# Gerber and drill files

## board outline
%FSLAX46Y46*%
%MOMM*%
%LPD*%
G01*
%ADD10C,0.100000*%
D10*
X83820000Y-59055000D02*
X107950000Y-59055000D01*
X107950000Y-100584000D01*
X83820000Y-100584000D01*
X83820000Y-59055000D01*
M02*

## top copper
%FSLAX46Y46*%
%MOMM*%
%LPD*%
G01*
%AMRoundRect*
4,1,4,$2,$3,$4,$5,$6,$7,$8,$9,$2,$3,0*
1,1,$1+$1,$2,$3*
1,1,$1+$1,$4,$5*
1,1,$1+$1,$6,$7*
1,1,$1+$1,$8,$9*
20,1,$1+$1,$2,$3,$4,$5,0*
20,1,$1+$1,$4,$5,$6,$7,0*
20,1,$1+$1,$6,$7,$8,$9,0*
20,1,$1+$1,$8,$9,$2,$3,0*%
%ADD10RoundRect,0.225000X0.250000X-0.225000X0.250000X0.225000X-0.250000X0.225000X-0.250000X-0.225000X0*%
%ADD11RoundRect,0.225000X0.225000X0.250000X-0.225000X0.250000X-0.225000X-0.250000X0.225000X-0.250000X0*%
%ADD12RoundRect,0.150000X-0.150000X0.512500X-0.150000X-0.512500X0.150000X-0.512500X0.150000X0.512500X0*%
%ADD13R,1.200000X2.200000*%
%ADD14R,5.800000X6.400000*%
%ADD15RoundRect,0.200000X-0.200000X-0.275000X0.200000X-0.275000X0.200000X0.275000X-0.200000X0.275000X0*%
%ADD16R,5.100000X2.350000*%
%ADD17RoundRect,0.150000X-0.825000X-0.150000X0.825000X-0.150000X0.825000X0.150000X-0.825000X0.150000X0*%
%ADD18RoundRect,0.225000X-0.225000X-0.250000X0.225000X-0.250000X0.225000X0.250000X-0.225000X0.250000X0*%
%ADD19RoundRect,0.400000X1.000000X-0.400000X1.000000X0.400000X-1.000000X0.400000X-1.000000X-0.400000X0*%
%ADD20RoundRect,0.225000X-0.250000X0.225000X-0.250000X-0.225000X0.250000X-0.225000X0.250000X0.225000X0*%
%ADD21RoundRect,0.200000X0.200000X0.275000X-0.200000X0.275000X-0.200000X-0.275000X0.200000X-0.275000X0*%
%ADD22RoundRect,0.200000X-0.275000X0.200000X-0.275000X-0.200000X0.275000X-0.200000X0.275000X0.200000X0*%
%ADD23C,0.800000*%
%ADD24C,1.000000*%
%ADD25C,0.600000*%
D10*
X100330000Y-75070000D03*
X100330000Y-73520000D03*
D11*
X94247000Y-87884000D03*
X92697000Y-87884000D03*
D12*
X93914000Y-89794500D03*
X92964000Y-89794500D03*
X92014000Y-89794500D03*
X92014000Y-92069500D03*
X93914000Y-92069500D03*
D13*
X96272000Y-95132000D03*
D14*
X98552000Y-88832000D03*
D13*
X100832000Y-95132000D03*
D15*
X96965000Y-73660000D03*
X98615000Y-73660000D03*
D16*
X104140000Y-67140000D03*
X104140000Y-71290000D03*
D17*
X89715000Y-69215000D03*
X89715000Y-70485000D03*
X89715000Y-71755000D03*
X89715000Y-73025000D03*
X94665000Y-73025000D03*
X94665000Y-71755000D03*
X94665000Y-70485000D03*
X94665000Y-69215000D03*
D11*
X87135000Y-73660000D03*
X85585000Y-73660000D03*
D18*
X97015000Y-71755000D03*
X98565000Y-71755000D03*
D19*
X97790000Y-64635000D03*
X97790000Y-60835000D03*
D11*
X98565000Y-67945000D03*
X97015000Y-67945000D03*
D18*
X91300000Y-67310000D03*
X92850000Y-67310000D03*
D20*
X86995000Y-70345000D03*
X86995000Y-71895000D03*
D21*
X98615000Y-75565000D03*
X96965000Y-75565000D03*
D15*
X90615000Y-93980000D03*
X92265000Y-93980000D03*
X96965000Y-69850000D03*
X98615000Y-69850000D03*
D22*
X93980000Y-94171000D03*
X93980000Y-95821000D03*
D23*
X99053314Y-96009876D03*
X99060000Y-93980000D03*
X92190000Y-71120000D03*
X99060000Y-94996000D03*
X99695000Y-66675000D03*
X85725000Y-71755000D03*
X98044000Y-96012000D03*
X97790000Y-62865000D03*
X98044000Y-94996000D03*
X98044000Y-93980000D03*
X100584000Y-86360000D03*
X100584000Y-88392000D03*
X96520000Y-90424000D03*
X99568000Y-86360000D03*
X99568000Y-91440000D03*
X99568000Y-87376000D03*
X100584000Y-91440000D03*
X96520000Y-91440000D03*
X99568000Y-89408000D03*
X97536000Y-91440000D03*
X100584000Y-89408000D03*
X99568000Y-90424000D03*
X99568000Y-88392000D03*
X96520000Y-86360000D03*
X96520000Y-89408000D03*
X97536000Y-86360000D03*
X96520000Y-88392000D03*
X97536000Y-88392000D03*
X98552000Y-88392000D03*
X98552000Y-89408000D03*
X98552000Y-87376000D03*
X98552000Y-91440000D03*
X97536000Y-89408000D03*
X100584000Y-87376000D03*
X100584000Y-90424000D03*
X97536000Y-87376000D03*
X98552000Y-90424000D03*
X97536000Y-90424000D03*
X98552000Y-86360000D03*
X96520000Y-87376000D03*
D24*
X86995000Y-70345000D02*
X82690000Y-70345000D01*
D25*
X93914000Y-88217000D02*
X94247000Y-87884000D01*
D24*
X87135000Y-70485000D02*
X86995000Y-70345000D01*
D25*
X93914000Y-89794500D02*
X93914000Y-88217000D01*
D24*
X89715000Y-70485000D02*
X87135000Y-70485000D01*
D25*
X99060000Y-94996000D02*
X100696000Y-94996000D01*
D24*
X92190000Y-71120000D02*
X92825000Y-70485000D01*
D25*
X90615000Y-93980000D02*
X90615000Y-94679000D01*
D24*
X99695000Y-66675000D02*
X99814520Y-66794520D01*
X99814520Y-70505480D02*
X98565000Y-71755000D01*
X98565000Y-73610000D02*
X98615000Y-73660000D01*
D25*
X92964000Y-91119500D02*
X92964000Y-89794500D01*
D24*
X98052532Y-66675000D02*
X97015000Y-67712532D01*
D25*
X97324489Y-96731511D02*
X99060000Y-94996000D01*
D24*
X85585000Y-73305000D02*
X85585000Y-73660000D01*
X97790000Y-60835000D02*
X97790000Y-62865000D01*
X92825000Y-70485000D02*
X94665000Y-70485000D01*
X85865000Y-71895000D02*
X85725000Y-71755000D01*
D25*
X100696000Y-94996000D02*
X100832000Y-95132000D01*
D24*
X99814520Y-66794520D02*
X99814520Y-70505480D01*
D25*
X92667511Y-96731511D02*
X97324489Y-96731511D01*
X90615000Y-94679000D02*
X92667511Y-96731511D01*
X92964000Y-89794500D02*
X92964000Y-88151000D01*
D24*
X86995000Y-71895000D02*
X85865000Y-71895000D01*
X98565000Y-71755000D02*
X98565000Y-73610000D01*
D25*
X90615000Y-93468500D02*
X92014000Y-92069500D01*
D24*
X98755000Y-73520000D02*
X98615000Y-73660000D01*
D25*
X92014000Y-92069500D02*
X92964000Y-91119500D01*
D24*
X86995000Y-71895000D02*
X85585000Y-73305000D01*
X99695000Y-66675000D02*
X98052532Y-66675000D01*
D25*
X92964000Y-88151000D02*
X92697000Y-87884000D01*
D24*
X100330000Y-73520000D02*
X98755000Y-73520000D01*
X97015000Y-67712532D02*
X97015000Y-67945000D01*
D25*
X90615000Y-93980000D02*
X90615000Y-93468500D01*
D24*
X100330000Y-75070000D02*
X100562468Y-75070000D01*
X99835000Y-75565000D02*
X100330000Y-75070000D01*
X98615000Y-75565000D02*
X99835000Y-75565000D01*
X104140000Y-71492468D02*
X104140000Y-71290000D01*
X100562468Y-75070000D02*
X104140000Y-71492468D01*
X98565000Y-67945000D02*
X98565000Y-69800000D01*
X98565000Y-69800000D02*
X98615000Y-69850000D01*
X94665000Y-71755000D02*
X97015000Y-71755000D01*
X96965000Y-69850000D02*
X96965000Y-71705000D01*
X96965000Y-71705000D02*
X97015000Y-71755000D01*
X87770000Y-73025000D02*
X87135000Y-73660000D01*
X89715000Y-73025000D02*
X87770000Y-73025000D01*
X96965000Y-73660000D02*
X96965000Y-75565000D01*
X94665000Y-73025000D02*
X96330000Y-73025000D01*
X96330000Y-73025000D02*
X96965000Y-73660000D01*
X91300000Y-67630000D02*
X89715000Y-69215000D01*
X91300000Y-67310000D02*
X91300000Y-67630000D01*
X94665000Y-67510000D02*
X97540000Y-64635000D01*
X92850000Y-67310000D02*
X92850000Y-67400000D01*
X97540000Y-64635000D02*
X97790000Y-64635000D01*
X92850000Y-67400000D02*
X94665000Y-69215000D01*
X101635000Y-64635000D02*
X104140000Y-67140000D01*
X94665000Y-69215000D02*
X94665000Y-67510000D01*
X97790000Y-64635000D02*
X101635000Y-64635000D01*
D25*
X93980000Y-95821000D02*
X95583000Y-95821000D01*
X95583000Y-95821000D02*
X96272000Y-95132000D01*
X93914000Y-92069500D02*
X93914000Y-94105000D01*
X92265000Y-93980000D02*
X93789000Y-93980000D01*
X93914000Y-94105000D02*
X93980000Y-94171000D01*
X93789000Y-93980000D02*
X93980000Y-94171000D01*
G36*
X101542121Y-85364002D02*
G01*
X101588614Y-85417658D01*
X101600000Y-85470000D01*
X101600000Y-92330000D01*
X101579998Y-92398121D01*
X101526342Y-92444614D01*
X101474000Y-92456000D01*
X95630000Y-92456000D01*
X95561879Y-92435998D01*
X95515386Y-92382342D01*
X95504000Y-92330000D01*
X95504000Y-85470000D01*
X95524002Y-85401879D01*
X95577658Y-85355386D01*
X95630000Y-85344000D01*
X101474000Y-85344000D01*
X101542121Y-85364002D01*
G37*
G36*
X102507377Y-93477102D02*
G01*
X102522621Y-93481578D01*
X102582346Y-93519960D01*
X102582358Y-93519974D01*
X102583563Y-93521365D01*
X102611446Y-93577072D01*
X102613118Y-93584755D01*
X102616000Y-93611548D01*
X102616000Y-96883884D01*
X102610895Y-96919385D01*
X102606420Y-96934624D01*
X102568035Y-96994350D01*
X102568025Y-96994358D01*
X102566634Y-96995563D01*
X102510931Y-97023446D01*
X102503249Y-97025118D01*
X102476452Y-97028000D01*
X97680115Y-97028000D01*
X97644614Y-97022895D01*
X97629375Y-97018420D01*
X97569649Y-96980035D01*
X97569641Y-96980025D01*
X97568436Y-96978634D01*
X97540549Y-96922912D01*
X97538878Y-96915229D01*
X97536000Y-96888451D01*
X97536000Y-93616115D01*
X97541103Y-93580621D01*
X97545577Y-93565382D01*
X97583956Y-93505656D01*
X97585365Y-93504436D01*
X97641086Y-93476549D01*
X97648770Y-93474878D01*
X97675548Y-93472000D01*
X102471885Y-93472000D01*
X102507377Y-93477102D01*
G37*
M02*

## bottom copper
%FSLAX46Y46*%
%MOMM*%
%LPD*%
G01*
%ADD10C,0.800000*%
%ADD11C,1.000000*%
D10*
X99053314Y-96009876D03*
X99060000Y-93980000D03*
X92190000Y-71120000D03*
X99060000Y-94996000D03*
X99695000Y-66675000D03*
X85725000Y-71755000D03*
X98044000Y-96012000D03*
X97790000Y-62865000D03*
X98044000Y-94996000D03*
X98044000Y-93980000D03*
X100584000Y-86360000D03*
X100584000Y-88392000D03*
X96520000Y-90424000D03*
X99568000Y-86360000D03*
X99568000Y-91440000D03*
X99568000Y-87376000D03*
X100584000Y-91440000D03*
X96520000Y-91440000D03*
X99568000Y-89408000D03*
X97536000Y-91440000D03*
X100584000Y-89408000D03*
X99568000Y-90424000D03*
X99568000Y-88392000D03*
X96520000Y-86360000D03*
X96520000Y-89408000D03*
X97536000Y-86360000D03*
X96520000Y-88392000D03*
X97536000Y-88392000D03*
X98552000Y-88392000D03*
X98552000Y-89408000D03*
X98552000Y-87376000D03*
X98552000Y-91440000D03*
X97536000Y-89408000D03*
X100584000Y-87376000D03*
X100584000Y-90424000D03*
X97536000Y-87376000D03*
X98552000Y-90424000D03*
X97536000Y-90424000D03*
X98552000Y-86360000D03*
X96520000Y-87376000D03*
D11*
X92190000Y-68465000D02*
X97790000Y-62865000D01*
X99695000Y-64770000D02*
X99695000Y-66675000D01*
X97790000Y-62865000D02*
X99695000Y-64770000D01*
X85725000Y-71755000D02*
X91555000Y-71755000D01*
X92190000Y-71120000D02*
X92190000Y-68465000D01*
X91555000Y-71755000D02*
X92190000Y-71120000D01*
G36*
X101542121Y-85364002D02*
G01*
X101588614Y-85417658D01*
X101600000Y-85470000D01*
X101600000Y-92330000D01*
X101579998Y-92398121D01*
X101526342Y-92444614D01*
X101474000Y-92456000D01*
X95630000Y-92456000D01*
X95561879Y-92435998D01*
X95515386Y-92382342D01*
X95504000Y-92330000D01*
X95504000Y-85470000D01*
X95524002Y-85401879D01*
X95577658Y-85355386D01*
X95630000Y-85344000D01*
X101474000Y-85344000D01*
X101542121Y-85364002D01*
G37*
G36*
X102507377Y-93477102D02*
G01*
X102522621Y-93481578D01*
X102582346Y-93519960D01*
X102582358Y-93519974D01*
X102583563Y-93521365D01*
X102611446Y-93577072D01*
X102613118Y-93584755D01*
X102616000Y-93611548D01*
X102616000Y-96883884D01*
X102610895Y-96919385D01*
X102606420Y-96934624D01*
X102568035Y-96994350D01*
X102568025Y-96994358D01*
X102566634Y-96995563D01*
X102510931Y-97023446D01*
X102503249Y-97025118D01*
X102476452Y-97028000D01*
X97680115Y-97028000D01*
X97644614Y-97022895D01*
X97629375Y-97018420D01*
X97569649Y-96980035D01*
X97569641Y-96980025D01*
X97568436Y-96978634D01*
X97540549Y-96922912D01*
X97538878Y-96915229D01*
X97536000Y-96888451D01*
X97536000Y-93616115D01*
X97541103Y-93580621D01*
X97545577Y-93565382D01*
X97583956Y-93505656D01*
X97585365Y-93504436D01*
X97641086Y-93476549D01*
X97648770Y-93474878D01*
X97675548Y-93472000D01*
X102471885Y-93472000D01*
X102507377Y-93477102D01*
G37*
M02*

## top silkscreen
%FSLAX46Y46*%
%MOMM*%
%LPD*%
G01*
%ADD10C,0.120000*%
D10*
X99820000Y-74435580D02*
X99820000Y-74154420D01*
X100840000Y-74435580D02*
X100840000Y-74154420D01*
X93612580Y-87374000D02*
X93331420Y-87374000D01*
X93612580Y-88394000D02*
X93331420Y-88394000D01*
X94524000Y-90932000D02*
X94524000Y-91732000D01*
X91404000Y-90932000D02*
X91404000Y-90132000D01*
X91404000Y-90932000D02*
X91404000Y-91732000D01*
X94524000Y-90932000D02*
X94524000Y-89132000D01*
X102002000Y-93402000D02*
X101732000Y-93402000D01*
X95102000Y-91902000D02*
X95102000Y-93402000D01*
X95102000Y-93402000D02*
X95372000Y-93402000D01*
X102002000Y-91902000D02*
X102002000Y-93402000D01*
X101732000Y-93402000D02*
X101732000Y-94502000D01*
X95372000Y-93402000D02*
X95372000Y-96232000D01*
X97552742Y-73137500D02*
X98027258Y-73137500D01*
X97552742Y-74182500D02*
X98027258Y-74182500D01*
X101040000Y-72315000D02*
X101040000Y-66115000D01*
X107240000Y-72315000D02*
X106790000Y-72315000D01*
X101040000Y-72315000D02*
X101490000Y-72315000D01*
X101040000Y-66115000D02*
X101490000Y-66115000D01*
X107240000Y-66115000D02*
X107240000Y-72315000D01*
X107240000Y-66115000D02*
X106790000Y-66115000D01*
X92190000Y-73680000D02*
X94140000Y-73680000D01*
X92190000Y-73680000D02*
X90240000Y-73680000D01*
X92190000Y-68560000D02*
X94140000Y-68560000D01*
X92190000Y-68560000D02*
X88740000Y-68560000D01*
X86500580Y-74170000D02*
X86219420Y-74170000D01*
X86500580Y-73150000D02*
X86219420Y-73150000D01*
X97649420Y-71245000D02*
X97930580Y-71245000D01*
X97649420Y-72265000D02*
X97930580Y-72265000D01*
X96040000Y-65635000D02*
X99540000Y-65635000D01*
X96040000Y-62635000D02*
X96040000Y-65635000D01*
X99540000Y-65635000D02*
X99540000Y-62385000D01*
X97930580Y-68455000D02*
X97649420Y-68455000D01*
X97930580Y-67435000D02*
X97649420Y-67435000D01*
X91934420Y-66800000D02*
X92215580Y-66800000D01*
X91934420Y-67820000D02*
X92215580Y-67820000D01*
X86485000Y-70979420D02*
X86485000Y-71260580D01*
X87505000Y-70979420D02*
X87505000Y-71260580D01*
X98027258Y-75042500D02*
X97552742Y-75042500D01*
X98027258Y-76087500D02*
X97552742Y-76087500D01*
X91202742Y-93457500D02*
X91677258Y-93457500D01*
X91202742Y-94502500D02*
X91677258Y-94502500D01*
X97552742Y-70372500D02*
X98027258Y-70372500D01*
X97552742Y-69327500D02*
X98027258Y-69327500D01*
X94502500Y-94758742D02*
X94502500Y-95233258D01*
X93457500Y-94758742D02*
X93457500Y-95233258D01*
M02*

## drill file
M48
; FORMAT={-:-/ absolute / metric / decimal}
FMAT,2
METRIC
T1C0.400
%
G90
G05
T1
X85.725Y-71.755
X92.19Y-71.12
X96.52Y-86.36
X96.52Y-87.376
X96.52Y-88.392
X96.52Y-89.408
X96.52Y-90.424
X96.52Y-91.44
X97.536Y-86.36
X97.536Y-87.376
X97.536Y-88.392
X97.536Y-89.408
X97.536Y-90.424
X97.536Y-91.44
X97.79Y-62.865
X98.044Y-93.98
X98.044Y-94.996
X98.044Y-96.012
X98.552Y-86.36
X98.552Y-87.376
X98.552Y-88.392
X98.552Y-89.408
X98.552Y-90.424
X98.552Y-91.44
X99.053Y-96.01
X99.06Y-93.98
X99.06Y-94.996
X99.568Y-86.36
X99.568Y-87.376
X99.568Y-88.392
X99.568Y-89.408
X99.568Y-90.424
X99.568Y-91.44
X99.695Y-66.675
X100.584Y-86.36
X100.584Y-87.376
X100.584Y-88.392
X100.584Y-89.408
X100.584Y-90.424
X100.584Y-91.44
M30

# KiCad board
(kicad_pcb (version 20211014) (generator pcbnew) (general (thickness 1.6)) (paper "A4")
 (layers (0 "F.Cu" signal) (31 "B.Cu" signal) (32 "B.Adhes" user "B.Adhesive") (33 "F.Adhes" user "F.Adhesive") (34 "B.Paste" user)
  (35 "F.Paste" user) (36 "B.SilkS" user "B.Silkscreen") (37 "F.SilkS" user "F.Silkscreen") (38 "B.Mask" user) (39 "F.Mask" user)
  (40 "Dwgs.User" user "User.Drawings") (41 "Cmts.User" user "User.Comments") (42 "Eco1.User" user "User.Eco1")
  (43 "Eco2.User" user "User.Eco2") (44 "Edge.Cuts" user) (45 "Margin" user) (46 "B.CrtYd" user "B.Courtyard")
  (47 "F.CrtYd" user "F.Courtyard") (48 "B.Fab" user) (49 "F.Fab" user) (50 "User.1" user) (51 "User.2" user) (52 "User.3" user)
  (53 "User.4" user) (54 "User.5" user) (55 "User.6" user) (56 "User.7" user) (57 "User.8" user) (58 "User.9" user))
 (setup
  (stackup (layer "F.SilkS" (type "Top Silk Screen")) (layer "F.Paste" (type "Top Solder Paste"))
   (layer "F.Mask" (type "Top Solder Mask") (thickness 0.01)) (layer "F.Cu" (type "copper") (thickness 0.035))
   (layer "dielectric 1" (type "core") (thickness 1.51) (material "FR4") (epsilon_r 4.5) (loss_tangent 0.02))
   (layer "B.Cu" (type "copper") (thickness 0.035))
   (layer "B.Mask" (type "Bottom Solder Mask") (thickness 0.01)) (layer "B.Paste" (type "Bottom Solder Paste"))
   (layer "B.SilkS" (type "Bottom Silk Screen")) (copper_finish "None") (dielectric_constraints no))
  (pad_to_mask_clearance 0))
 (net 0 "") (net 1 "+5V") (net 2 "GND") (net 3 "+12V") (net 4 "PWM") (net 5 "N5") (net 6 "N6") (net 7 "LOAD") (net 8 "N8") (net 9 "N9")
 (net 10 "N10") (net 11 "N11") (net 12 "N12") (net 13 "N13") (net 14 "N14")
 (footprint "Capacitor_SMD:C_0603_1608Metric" (layer "F.Cu") (at 100.33 74.295 90)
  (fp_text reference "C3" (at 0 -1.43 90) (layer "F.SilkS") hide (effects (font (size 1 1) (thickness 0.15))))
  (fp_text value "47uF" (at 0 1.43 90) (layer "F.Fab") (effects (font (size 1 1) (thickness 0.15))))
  (fp_line (start -0.14058 -0.51) (end 0.14058 -0.51) (layer "F.SilkS") (width 0.12))
  (fp_line (start -0.14058 0.51) (end 0.14058 0.51) (layer "F.SilkS") (width 0.12))
  (pad "1" smd roundrect (at -0.775 0 90) (size 0.9 0.95) (layers "F.Cu" "F.Paste" "F.Mask") (roundrect_rratio 0.25) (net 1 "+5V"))
  (pad "2" smd roundrect (at 0.775 0 90) (size 0.9 0.95) (layers "F.Cu" "F.Paste" "F.Mask") (roundrect_rratio 0.25) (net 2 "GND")))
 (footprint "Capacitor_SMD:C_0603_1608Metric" (layer "F.Cu") (at 93.472 87.884 180)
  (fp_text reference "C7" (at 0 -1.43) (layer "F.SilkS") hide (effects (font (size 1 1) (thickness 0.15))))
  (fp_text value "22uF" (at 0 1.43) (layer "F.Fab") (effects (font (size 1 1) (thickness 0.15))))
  (fp_line (start -0.14058 0.51) (end 0.14058 0.51) (layer "F.SilkS") (width 0.12))
  (fp_line (start -0.14058 -0.51) (end 0.14058 -0.51) (layer "F.SilkS") (width 0.12))
  (pad "1" smd roundrect (at -0.775 0 180) (size 0.9 0.95) (layers "F.Cu" "F.Paste" "F.Mask") (roundrect_rratio 0.25) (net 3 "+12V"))
  (pad "2" smd roundrect (at 0.775 0 180) (size 0.9 0.95) (layers "F.Cu" "F.Paste" "F.Mask") (roundrect_rratio 0.25) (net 2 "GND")))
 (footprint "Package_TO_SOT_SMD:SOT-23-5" (layer "F.Cu") (at 92.964 90.932 -90)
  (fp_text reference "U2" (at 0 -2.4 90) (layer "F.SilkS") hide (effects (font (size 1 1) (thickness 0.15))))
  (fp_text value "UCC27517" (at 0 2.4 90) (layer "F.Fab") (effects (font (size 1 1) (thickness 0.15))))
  (fp_line (start 0 -1.56) (end 0.8 -1.56) (layer "F.SilkS") (width 0.12))
  (fp_line (start 0 1.56) (end -0.8 1.56) (layer "F.SilkS") (width 0.12))
  (fp_line (start 0 1.56) (end 0.8 1.56) (layer "F.SilkS") (width 0.12))
  (fp_line (start 0 -1.56) (end -1.8 -1.56) (layer "F.SilkS") (width 0.12))
  (pad "1" smd roundrect (at -1.1375 -0.95 270) (size 1.325 0.6) (layers "F.Cu" "F.Paste" "F.Mask") (roundrect_rratio 0.25) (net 3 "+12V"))
  (pad "2" smd roundrect (at -1.1375 0 270) (size 1.325 0.6) (layers "F.Cu" "F.Paste" "F.Mask") (roundrect_rratio 0.25) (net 2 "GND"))
  (pad "3" smd roundrect (at -1.1375 0.95 270) (size 1.325 0.6) (layers "F.Cu" "F.Paste" "F.Mask") (roundrect_rratio 0.25) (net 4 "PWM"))
  (pad "4" smd roundrect (at 1.1375 0.95 270) (size 1.325 0.6) (layers "F.Cu" "F.Paste" "F.Mask") (roundrect_rratio 0.25) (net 2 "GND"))
  (pad "5" smd roundrect (at 1.1375 -0.95 270) (size 1.325 0.6) (layers "F.Cu" "F.Paste" "F.Mask") (roundrect_rratio 0.25) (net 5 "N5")))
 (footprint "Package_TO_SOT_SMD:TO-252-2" (layer "F.Cu") (at 98.552 90.932 90)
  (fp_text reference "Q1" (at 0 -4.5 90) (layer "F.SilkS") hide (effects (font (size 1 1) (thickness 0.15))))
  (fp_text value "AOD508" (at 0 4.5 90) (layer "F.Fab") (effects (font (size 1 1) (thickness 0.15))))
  (fp_line (start -2.47 3.45) (end -2.47 3.18) (layer "F.SilkS") (width 0.12))
  (fp_line (start -0.97 -3.45) (end -2.47 -3.45) (layer "F.SilkS") (width 0.12))
  (fp_line (start -2.47 -3.45) (end -2.47 -3.18) (layer "F.SilkS") (width 0.12))
  (fp_line (start -0.97 3.45) (end -2.47 3.45) (layer "F.SilkS") (width 0.12))
  (fp_line (start -2.47 3.18) (end -3.57 3.18) (layer "F.SilkS") (width 0.12))
  (fp_line (start -2.47 -3.18) (end -5.3 -3.18) (layer "F.SilkS") (width 0.12))
  (pad "" smd rect (at 0.425 1.525 90) (size 3.05 2.75) (layers "F.Paste"))
  (pad "" smd rect (at 3.775 1.525 90) (size 3.05 2.75) (layers "F.Paste"))
  (pad "" smd rect (at 3.775 -1.525 90) (size 3.05 2.75) (layers "F.Paste"))
  (pad "" smd rect (at 0.425 -1.525 90) (size 3.05 2.75) (layers "F.Paste"))
  (pad "1" smd rect (at -4.2 -2.28 90) (size 2.2 1.2) (layers "F.Cu" "F.Paste" "F.Mask") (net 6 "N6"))
  (pad "2" smd rect (at 2.1 0 90) (size 6.4 5.8) (layers "F.Cu" "F.Mask") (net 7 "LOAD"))
  (pad "3" smd rect (at -4.2 2.28 90) (size 2.2 1.2) (layers "F.Cu" "F.Paste" "F.Mask") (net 2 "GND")))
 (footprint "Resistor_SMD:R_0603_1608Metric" (layer "F.Cu") (at 97.79 73.66)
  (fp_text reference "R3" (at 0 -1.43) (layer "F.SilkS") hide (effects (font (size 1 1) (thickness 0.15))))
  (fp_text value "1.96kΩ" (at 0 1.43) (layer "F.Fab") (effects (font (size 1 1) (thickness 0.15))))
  (fp_line (start -0.237258 -0.5225) (end 0.237258 -0.5225) (layer "F.SilkS") (width 0.12))
  (fp_line (start -0.237258 0.5225) (end 0.237258 0.5225) (layer "F.SilkS") (width 0.12))
  (pad "1" smd roundrect (at -0.825 0) (size 0.8 0.95) (layers "F.Cu" "F.Paste" "F.Mask") (roundrect_rratio 0.25) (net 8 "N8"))
  (pad "2" smd roundrect (at 0.825 0) (size 0.8 0.95) (layers "F.Cu" "F.Paste" "F.Mask") (roundrect_rratio 0.25) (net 2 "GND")))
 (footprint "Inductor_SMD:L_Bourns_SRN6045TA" (layer "F.Cu") (at 104.14 69.215 -90)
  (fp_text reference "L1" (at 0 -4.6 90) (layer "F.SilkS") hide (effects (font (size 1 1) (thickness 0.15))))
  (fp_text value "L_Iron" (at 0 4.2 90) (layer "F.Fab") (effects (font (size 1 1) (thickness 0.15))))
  (fp_line (start 3.1 3.1) (end -3.1 3.1) (layer "F.SilkS") (width 0.12))
  (fp_line (start 3.1 -3.1) (end 3.1 -2.65) (layer "F.SilkS") (width 0.12))
  (fp_line (start 3.1 3.1) (end 3.1 2.65) (layer "F.SilkS") (width 0.12))
  (fp_line (start -3.1 3.1) (end -3.1 2.65) (layer "F.SilkS") (width 0.12))
  (fp_line (start -3.1 -3.1) (end 3.1 -3.1) (layer "F.SilkS") (width 0.12))
  (fp_line (start -3.1 -3.1) (end -3.1 -2.65) (layer "F.SilkS") (width 0.12))
  (pad "1" smd rect (at -2.075 0 270) (size 2.35 5.1) (layers "F.Cu" "F.Paste" "F.Mask") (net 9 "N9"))
  (pad "2" smd rect (at 2.075 0 270) (size 2.35 5.1) (layers "F.Cu" "F.Paste" "F.Mask") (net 1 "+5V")))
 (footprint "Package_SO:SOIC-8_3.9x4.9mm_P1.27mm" (layer "F.Cu") (at 92.19 71.12)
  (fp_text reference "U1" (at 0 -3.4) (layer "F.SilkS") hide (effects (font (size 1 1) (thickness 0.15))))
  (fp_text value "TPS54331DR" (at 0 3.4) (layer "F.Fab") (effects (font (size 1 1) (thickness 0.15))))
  (fp_line (start 0 2.56) (end 1.95 2.56) (layer "F.SilkS") (width 0.12))
  (fp_line (start 0 2.56) (end -1.95 2.56) (layer "F.SilkS") (width 0.12))
  (fp_line (start 0 -2.56) (end 1.95 -2.56) (layer "F.SilkS") (width 0.12))
  (fp_line (start 0 -2.56) (end -3.45 -2.56) (layer "F.SilkS") (width 0.12))
  (pad "1" smd roundrect (at -2.475 -1.905) (size 1.95 0.6) (layers "F.Cu" "F.Paste" "F.Mask") (roundrect_rratio 0.25) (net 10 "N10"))
  (pad "2" smd roundrect (at -2.475 -0.635) (size 1.95 0.6) (layers "F.Cu" "F.Paste" "F.Mask") (roundrect_rratio 0.25) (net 3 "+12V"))
  (pad "3" smd roundrect (at -2.475 0.635) (size 1.95 0.6) (layers "F.Cu" "F.Paste" "F.Mask") (roundrect_rratio 0.25) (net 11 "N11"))
  (pad "4" smd roundrect (at -2.475 1.905) (size 1.95 0.6) (layers "F.Cu" "F.Paste" "F.Mask") (roundrect_rratio 0.25) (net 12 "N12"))
  (pad "5" smd roundrect (at 2.475 1.905) (size 1.95 0.6) (layers "F.Cu" "F.Paste" "F.Mask") (roundrect_rratio 0.25) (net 8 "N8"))
  (pad "6" smd roundrect (at 2.475 0.635) (size 1.95 0.6) (layers "F.Cu" "F.Paste" "F.Mask") (roundrect_rratio 0.25) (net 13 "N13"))
  (pad "7" smd roundrect (at 2.475 -0.635) (size 1.95 0.6) (layers "F.Cu" "F.Paste" "F.Mask") (roundrect_rratio 0.25) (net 2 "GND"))
  (pad "8" smd roundrect (at 2.475 -1.905) (size 1.95 0.6) (layers "F.Cu" "F.Paste" "F.Mask") (roundrect_rratio 0.25) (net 9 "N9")))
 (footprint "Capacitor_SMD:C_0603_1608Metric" (layer "F.Cu") (at 86.36 73.66 180)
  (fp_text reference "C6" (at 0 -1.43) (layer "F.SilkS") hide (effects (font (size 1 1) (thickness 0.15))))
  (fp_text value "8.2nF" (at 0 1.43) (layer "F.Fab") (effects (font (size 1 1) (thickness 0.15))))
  (fp_line (start -0.14058 -0.51) (end 0.14058 -0.51) (layer "F.SilkS") (width 0.12))
  (fp_line (start -0.14058 0.51) (end 0.14058 0.51) (layer "F.SilkS") (width 0.12))
  (pad "1" smd roundrect (at -0.775 0 180) (size 0.9 0.95) (layers "F.Cu" "F.Paste" "F.Mask") (roundrect_rratio 0.25) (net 12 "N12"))
  (pad "2" smd roundrect (at 0.775 0 180) (size 0.9 0.95) (layers "F.Cu" "F.Paste" "F.Mask") (roundrect_rratio 0.25) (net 2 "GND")))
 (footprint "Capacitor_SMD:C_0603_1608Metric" (layer "F.Cu") (at 97.79 71.755)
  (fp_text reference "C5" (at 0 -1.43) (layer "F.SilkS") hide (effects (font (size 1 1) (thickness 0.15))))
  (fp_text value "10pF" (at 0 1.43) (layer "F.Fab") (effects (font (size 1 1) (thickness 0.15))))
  (fp_line (start -0.14058 -0.51) (end 0.14058 -0.51) (layer "F.SilkS") (width 0.12))
  (fp_line (start -0.14058 0.51) (end 0.14058 0.51) (layer "F.SilkS") (width 0.12))
  (pad "1" smd roundrect (at -0.775 0) (size 0.9 0.95) (layers "F.Cu" "F.Paste" "F.Mask") (roundrect_rratio 0.25) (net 13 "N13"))
  (pad "2" smd roundrect (at 0.775 0) (size 0.9 0.95) (layers "F.Cu" "F.Paste" "F.Mask") (roundrect_rratio 0.25) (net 2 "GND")))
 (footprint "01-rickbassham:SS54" (layer "F.Cu") (at 97.79 64.635 90)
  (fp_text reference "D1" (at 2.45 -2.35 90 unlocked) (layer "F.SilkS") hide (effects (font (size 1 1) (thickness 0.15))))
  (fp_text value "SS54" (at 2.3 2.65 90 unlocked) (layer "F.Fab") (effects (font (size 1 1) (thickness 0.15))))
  (fp_line (start -1 -1.75) (end -1 1.75) (layer "F.SilkS") (width 0.12))
  (fp_line (start 2 -1.75) (end -1 -1.75) (layer "F.SilkS") (width 0.12))
  (fp_line (start -1 1.75) (end 2.25 1.75) (layer "F.SilkS") (width 0.12))
  (pad "1" smd roundrect (at 0 0 90) (size 1.6 2.8) (layers "F.Cu" "F.Paste" "F.Mask") (roundrect_rratio 0.25) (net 9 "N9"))
  (pad "2" smd roundrect (at 3.8 0 90) (size 1.6 2.8) (layers "F.Cu" "F.Paste" "F.Mask") (roundrect_rratio 0.25) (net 2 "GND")))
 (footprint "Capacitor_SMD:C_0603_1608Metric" (layer "F.Cu") (at 97.79 67.945 180)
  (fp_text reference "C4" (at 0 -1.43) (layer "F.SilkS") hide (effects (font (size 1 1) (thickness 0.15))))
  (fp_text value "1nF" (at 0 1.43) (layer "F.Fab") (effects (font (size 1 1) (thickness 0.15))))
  (fp_line (start -0.14058 -0.51) (end 0.14058 -0.51) (layer "F.SilkS") (width 0.12))
  (fp_line (start -0.14058 0.51) (end 0.14058 0.51) (layer "F.SilkS") (width 0.12))
  (pad "1" smd roundrect (at -0.775 0 180) (size 0.9 0.95) (layers "F.Cu" "F.Paste" "F.Mask") (roundrect_rratio 0.25) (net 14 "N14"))
  (pad "2" smd roundrect (at 0.775 0 180) (size 0.9 0.95) (layers "F.Cu" "F.Paste" "F.Mask") (roundrect_rratio 0.25) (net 2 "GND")))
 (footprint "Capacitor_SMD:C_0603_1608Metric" (layer "F.Cu") (at 92.075 67.31)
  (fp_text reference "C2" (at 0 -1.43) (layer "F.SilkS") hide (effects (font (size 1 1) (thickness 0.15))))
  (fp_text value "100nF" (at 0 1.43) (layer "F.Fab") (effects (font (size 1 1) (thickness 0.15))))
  (fp_line (start -0.14058 -0.51) (end 0.14058 -0.51) (layer "F.SilkS") (width 0.12))
  (fp_line (start -0.14058 0.51) (end 0.14058 0.51) (layer "F.SilkS") (width 0.12))
  (pad "1" smd roundrect (at -0.775 0) (size 0.9 0.95) (layers "F.Cu" "F.Paste" "F.Mask") (roundrect_rratio 0.25) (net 10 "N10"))
  (pad "2" smd roundrect (at 0.775 0) (size 0.9 0.95) (layers "F.Cu" "F.Paste" "F.Mask") (roundrect_rratio 0.25) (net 9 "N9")))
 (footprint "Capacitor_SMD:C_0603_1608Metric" (layer "F.Cu") (at 86.995 71.12 -90)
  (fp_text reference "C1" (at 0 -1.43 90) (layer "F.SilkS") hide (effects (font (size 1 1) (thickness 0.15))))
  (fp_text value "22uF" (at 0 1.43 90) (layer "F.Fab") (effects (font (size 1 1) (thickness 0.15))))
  (fp_line (start -0.14058 0.51) (end 0.14058 0.51) (layer "F.SilkS") (width 0.12))
  (fp_line (start -0.14058 -0.51) (end 0.14058 -0.51) (layer "F.SilkS") (width 0.12))
  (pad "1" smd roundrect (at -0.775 0 270) (size 0.9 0.95) (layers "F.Cu" "F.Paste" "F.Mask") (roundrect_rratio 0.25) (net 3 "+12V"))
  (pad "2" smd roundrect (at 0.775 0 270) (size 0.9 0.95) (layers "F.Cu" "F.Paste" "F.Mask") (roundrect_rratio 0.25) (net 2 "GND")))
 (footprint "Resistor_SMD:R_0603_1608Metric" (layer "F.Cu") (at 97.79 75.565 180)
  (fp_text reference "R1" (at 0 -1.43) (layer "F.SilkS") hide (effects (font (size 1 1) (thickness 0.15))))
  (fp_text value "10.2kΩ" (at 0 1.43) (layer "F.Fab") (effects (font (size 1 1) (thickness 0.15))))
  (fp_line (start -0.237258 0.5225) (end 0.237258 0.5225) (layer "F.SilkS") (width 0.12))
  (fp_line (start -0.237258 -0.5225) (end 0.237258 -0.5225) (layer "F.SilkS") (width 0.12))
  (pad "1" smd roundrect (at -0.825 0 180) (size 0.8 0.95) (layers "F.Cu" "F.Paste" "F.Mask") (roundrect_rratio 0.25) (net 1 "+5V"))
  (pad "2" smd roundrect (at 0.825 0 180) (size 0.8 0.95) (layers "F.Cu" "F.Paste" "F.Mask") (roundrect_rratio 0.25) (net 8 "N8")))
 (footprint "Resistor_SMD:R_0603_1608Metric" (layer "F.Cu") (at 91.44 93.98)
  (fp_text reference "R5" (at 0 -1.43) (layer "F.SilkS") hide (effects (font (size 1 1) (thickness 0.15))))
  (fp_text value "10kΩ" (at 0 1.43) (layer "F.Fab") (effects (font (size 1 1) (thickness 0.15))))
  (fp_line (start -0.237258 -0.5225) (end 0.237258 -0.5225) (layer "F.SilkS") (width 0.12))
  (fp_line (start -0.237258 0.5225) (end 0.237258 0.5225) (layer "F.SilkS") (width 0.12))
  (pad "1" smd roundrect (at -0.825 0) (size 0.8 0.95) (layers "F.Cu" "F.Paste" "F.Mask") (roundrect_rratio 0.25) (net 2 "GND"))
  (pad "2" smd roundrect (at 0.825 0) (size 0.8 0.95) (layers "F.Cu" "F.Paste" "F.Mask") (roundrect_rratio 0.25) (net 5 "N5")))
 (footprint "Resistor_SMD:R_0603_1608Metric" (layer "F.Cu") (at 97.79 69.85)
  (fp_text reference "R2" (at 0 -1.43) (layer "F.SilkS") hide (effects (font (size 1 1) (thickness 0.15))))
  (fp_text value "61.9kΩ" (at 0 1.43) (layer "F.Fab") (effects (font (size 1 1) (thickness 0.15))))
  (fp_line (start -0.237258 0.5225) (end 0.237258 0.5225) (layer "F.SilkS") (width 0.12))
  (fp_line (start -0.237258 -0.5225) (end 0.237258 -0.5225) (layer "F.SilkS") (width 0.12))
  (pad "1" smd roundrect (at -0.825 0) (size 0.8 0.95) (layers "F.Cu" "F.Paste" "F.Mask") (roundrect_rratio 0.25) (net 13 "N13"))
  (pad "2" smd roundrect (at 0.825 0) (size 0.8 0.95) (layers "F.Cu" "F.Paste" "F.Mask") (roundrect_rratio 0.25) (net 14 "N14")))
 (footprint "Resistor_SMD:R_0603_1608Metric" (layer "F.Cu") (at 93.98 94.996 -90)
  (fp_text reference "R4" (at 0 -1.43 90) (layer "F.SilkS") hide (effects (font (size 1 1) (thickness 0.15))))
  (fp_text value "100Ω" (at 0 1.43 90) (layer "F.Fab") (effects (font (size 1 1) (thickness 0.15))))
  (fp_line (start -0.237258 -0.5225) (end 0.237258 -0.5225) (layer "F.SilkS") (width 0.12))
  (fp_line (start -0.237258 0.5225) (end 0.237258 0.5225) (layer "F.SilkS") (width 0.12))
  (pad "1" smd roundrect (at -0.825 0 270) (size 0.8 0.95) (layers "F.Cu" "F.Paste" "F.Mask") (roundrect_rratio 0.25) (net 5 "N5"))
  (pad "2" smd roundrect (at 0.825 0 270) (size 0.8 0.95) (layers "F.Cu" "F.Paste" "F.Mask") (roundrect_rratio 0.25) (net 6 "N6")))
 (gr_rect (start 83.82 59.055) (end 107.95 100.584) (layer "Edge.Cuts") (width 0.1) (fill none))
 (segment (start 86.995 70.345) (end 82.69 70.345) (width 1) (layer "F.Cu") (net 3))
 (segment (start 93.914 88.217) (end 94.247 87.884) (width 0.6) (layer "F.Cu") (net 3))
 (segment (start 87.135 70.485) (end 86.995 70.345) (width 1) (layer "F.Cu") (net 3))
 (segment (start 93.914 89.7945) (end 93.914 88.217) (width 0.6) (layer "F.Cu") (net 3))
 (segment (start 89.715 70.485) (end 87.135 70.485) (width 1) (layer "F.Cu") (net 3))
 (segment (start 99.06 94.996) (end 100.696 94.996) (width 0.6) (layer "F.Cu") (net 2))
 (segment (start 92.19 71.12) (end 92.825 70.485) (width 1) (layer "F.Cu") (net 2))
 (segment (start 90.615 93.98) (end 90.615 94.679) (width 0.6) (layer "F.Cu") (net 2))
 (segment (start 99.695 66.675) (end 99.81452 66.79452) (width 1) (layer "F.Cu") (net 2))
 (segment (start 99.81452 70.50548) (end 98.565 71.755) (width 1) (layer "F.Cu") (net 2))
 (segment (start 98.565 73.61) (end 98.615 73.66) (width 1) (layer "F.Cu") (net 2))
 (segment (start 92.964 91.1195) (end 92.964 89.7945) (width 0.6) (layer "F.Cu") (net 2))
 (segment (start 98.052532 66.675) (end 97.015 67.712532) (width 1) (layer "F.Cu") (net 2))
 (segment (start 97.324489 96.731511) (end 99.06 94.996) (width 0.6) (layer "F.Cu") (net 2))
 (segment (start 85.585 73.305) (end 85.585 73.66) (width 1) (layer "F.Cu") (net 2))
 (segment (start 97.79 60.835) (end 97.79 62.865) (width 1) (layer "F.Cu") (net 2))
 (segment (start 92.825 70.485) (end 94.665 70.485) (width 1) (layer "F.Cu") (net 2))
 (segment (start 85.865 71.895) (end 85.725 71.755) (width 1) (layer "F.Cu") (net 2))
 (segment (start 100.696 94.996) (end 100.832 95.132) (width 0.6) (layer "F.Cu") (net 2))
 (segment (start 99.81452 66.79452) (end 99.81452 70.50548) (width 1) (layer "F.Cu") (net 2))
 (segment (start 92.667511 96.731511) (end 97.324489 96.731511) (width 0.6) (layer "F.Cu") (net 2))
 (segment (start 90.615 94.679) (end 92.667511 96.731511) (width 0.6) (layer "F.Cu") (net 2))
 (segment (start 92.964 89.7945) (end 92.964 88.151) (width 0.6) (layer "F.Cu") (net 2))
 (segment (start 86.995 71.895) (end 85.865 71.895) (width 1) (layer "F.Cu") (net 2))
 (segment (start 98.565 71.755) (end 98.565 73.61) (width 1) (layer "F.Cu") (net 2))
 (segment (start 90.615 93.4685) (end 92.014 92.0695) (width 0.6) (layer "F.Cu") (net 2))
 (segment (start 98.755 73.52) (end 98.615 73.66) (width 1) (layer "F.Cu") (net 2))
 (segment (start 92.014 92.0695) (end 92.964 91.1195) (width 0.6) (layer "F.Cu") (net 2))
 (segment (start 86.995 71.895) (end 85.585 73.305) (width 1) (layer "F.Cu") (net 2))
 (segment (start 99.695 66.675) (end 98.052532 66.675) (width 1) (layer "F.Cu") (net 2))
 (segment (start 92.964 88.151) (end 92.697 87.884) (width 0.6) (layer "F.Cu") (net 2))
 (segment (start 100.33 73.52) (end 98.755 73.52) (width 1) (layer "F.Cu") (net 2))
 (segment (start 97.015 67.712532) (end 97.015 67.945) (width 1) (layer "F.Cu") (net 2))
 (segment (start 90.615 93.98) (end 90.615 93.4685) (width 0.6) (layer "F.Cu") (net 2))
 (via (at 99.053314 96.009876) (size 0.8) (drill 0.4) (layers "F.Cu" "B.Cu") (free) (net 2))
 (via (at 99.06 93.98) (size 0.8) (drill 0.4) (layers "F.Cu" "B.Cu") (free) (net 2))
 (via (at 92.19 71.12) (size 0.8) (drill 0.4) (layers "F.Cu" "B.Cu") (free) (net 2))
 (via (at 99.06 94.996) (size 0.8) (drill 0.4) (layers "F.Cu" "B.Cu") (free) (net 2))
 (via (at 99.695 66.675) (size 0.8) (drill 0.4) (layers "F.Cu" "B.Cu") (free) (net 2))
 (via (at 85.725 71.755) (size 0.8) (drill 0.4) (layers "F.Cu" "B.Cu") (free) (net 2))
 (via (at 98.044 96.012) (size 0.8) (drill 0.4) (layers "F.Cu" "B.Cu") (free) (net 2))
 (via (at 97.79 62.865) (size 0.8) (drill 0.4) (layers "F.Cu" "B.Cu") (free) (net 2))
 (via (at 98.044 94.996) (size 0.8) (drill 0.4) (layers "F.Cu" "B.Cu") (free) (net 2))
 (via (at 98.044 93.98) (size 0.8) (drill 0.4) (layers "F.Cu" "B.Cu") (free) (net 2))
 (segment (start 92.19 68.465) (end 97.79 62.865) (width 1) (layer "B.Cu") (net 2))
 (segment (start 99.695 64.77) (end 99.695 66.675) (width 1) (layer "B.Cu") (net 2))
 (segment (start 97.79 62.865) (end 99.695 64.77) (width 1) (layer "B.Cu") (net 2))
 (segment (start 85.725 71.755) (end 91.555 71.755) (width 1) (layer "B.Cu") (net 2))
 (segment (start 92.19 71.12) (end 92.19 68.465) (width 1) (layer "B.Cu") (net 2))
 (segment (start 91.555 71.755) (end 92.19 71.12) (width 1) (layer "B.Cu") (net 2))
 (segment (start 100.33 75.07) (end 100.562468 75.07) (width 1) (layer "F.Cu") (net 1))
 (segment (start 99.835 75.565) (end 100.33 75.07) (width 1) (layer "F.Cu") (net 1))
 (segment (start 98.615 75.565) (end 99.835 75.565) (width 1) (layer "F.Cu") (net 1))
 (segment (start 104.14 71.492468) (end 104.14 71.29) (width 1) (layer "F.Cu") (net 1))
 (segment (start 100.562468 75.07) (end 104.14 71.492468) (width 1) (layer "F.Cu") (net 1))
 (segment (start 98.565 67.945) (end 98.565 69.8) (width 1) (layer "F.Cu") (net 14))
 (segment (start 98.565 69.8) (end 98.615 69.85) (width 1) (layer "F.Cu") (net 14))
 (segment (start 94.665 71.755) (end 97.015 71.755) (width 1) (layer "F.Cu") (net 13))
 (segment (start 96.965 69.85) (end 96.965 71.705) (width 1) (layer "F.Cu") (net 13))
 (segment (start 96.965 71.705) (end 97.015 71.755) (width 1) (layer "F.Cu") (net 13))
 (segment (start 87.77 73.025) (end 87.135 73.66) (width 1) (layer "F.Cu") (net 12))
 (segment (start 89.715 73.025) (end 87.77 73.025) (width 1) (layer "F.Cu") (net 12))
 (segment (start 96.965 73.66) (end 96.965 75.565) (width 1) (layer "F.Cu") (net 8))
 (segment (start 94.665 73.025) (end 96.33 73.025) (width 1) (layer "F.Cu") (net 8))
 (segment (start 96.33 73.025) (end 96.965 73.66) (width 1) (layer "F.Cu") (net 8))
 (segment (start 91.3 67.63) (end 89.715 69.215) (width 1) (layer "F.Cu") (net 10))
 (segment (start 91.3 67.31) (end 91.3 67.63) (width 1) (layer "F.Cu") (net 10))
 (segment (start 94.665 67.51) (end 97.54 64.635) (width 1) (layer "F.Cu") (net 9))
 (segment (start 92.85 67.31) (end 92.85 67.4) (width 1) (layer "F.Cu") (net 9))
 (segment (start 97.54 64.635) (end 97.79 64.635) (width 1) (layer "F.Cu") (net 9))
 (segment (start 92.85 67.4) (end 94.665 69.215) (width 1) (layer "F.Cu") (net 9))
 (segment (start 101.635 64.635) (end 104.14 67.14) (width 1) (layer "F.Cu") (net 9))
 (segment (start 94.665 69.215) (end 94.665 67.51) (width 1) (layer "F.Cu") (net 9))
 (segment (start 97.79 64.635) (end 101.635 64.635) (width 1) (layer "F.Cu") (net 9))
 (segment (start 93.98 95.821) (end 95.583 95.821) (width 0.6) (layer "F.Cu") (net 6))
 (segment (start 95.583 95.821) (end 96.272 95.132) (width 0.6) (layer "F.Cu") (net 6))
 (segment (start 93.914 92.0695) (end 93.914 94.105) (width 0.6) (layer "F.Cu") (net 5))
 (segment (start 92.265 93.98) (end 93.789 93.98) (width 0.6) (layer "F.Cu") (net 5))
 (segment (start 93.914 94.105) (end 93.98 94.171) (width 0.6) (layer "F.Cu") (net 5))
 (segment (start 93.789 93.98) (end 93.98 94.171) (width 0.6) (layer "F.Cu") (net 5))
 (via (at 100.584 86.36) (size 0.8) (drill 0.4) (layers "F.Cu" "B.Cu") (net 7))
 (via (at 100.584 88.392) (size 0.8) (drill 0.4) (layers "F.Cu" "B.Cu") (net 7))
 (via (at 96.52 90.424) (size 0.8) (drill 0.4) (layers "F.Cu" "B.Cu") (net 7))
 (via (at 99.568 86.36) (size 0.8) (drill 0.4) (layers "F.Cu" "B.Cu") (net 7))
 (via (at 99.568 91.44) (size 0.8) (drill 0.4) (layers "F.Cu" "B.Cu") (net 7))
 (via (at 99.568 87.376) (size 0.8) (drill 0.4) (layers "F.Cu" "B.Cu") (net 7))
 (via (at 100.584 91.44) (size 0.8) (drill 0.4) (layers "F.Cu" "B.Cu") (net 7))
 (via (at 96.52 91.44) (size 0.8) (drill 0.4) (layers "F.Cu" "B.Cu") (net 7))
 (via (at 99.568 89.408) (size 0.8) (drill 0.4) (layers "F.Cu" "B.Cu") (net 7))
 (via (at 97.536 91.44) (size 0.8) (drill 0.4) (layers "F.Cu" "B.Cu") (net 7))
 (via (at 100.584 89.408) (size 0.8) (drill 0.4) (layers "F.Cu" "B.Cu") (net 7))
 (via (at 99.568 90.424) (size 0.8) (drill 0.4) (layers "F.Cu" "B.Cu") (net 7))
 (via (at 99.568 88.392) (size 0.8) (drill 0.4) (layers "F.Cu" "B.Cu") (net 7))
 (via (at 96.52 86.36) (size 0.8) (drill 0.4) (layers "F.Cu" "B.Cu") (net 7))
 (via (at 96.52 89.408) (size 0.8) (drill 0.4) (layers "F.Cu" "B.Cu") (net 7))
 (via (at 97.536 86.36) (size 0.8) (drill 0.4) (layers "F.Cu" "B.Cu") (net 7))
 (via (at 96.52 88.392) (size 0.8) (drill 0.4) (layers "F.Cu" "B.Cu") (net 7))
 (via (at 97.536 88.392) (size 0.8) (drill 0.4) (layers "F.Cu" "B.Cu") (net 7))
 (via (at 98.552 88.392) (size 0.8) (drill 0.4) (layers "F.Cu" "B.Cu") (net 7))
 (via (at 98.552 89.408) (size 0.8) (drill 0.4) (layers "F.Cu" "B.Cu") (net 7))
 (via (at 98.552 87.376) (size 0.8) (drill 0.4) (layers "F.Cu" "B.Cu") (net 7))
 (via (at 98.552 91.44) (size 0.8) (drill 0.4) (layers "F.Cu" "B.Cu") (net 7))
 (via (at 97.536 89.408) (size 0.8) (drill 0.4) (layers "F.Cu" "B.Cu") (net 7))
 (via (at 100.584 87.376) (size 0.8) (drill 0.4) (layers "F.Cu" "B.Cu") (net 7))
 (via (at 100.584 90.424) (size 0.8) (drill 0.4) (layers "F.Cu" "B.Cu") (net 7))
 (via (at 97.536 87.376) (size 0.8) (drill 0.4) (layers "F.Cu" "B.Cu") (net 7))
 (via (at 98.552 90.424) (size 0.8) (drill 0.4) (layers "F.Cu" "B.Cu") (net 7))
 (via (at 97.536 90.424) (size 0.8) (drill 0.4) (layers "F.Cu" "B.Cu") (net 7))
 (via (at 98.552 86.36) (size 0.8) (drill 0.4) (layers "F.Cu" "B.Cu") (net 7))
 (via (at 96.52 87.376) (size 0.8) (drill 0.4) (layers "F.Cu" "B.Cu") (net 7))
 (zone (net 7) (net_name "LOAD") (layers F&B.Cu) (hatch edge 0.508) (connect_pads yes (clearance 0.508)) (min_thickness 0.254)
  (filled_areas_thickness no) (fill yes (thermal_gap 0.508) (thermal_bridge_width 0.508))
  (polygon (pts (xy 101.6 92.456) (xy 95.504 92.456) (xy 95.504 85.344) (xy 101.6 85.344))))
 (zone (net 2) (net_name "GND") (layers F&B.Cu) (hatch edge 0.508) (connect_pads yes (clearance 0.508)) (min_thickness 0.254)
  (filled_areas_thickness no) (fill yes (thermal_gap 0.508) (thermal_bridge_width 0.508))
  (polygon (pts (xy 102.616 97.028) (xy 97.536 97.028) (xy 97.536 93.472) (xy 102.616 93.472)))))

